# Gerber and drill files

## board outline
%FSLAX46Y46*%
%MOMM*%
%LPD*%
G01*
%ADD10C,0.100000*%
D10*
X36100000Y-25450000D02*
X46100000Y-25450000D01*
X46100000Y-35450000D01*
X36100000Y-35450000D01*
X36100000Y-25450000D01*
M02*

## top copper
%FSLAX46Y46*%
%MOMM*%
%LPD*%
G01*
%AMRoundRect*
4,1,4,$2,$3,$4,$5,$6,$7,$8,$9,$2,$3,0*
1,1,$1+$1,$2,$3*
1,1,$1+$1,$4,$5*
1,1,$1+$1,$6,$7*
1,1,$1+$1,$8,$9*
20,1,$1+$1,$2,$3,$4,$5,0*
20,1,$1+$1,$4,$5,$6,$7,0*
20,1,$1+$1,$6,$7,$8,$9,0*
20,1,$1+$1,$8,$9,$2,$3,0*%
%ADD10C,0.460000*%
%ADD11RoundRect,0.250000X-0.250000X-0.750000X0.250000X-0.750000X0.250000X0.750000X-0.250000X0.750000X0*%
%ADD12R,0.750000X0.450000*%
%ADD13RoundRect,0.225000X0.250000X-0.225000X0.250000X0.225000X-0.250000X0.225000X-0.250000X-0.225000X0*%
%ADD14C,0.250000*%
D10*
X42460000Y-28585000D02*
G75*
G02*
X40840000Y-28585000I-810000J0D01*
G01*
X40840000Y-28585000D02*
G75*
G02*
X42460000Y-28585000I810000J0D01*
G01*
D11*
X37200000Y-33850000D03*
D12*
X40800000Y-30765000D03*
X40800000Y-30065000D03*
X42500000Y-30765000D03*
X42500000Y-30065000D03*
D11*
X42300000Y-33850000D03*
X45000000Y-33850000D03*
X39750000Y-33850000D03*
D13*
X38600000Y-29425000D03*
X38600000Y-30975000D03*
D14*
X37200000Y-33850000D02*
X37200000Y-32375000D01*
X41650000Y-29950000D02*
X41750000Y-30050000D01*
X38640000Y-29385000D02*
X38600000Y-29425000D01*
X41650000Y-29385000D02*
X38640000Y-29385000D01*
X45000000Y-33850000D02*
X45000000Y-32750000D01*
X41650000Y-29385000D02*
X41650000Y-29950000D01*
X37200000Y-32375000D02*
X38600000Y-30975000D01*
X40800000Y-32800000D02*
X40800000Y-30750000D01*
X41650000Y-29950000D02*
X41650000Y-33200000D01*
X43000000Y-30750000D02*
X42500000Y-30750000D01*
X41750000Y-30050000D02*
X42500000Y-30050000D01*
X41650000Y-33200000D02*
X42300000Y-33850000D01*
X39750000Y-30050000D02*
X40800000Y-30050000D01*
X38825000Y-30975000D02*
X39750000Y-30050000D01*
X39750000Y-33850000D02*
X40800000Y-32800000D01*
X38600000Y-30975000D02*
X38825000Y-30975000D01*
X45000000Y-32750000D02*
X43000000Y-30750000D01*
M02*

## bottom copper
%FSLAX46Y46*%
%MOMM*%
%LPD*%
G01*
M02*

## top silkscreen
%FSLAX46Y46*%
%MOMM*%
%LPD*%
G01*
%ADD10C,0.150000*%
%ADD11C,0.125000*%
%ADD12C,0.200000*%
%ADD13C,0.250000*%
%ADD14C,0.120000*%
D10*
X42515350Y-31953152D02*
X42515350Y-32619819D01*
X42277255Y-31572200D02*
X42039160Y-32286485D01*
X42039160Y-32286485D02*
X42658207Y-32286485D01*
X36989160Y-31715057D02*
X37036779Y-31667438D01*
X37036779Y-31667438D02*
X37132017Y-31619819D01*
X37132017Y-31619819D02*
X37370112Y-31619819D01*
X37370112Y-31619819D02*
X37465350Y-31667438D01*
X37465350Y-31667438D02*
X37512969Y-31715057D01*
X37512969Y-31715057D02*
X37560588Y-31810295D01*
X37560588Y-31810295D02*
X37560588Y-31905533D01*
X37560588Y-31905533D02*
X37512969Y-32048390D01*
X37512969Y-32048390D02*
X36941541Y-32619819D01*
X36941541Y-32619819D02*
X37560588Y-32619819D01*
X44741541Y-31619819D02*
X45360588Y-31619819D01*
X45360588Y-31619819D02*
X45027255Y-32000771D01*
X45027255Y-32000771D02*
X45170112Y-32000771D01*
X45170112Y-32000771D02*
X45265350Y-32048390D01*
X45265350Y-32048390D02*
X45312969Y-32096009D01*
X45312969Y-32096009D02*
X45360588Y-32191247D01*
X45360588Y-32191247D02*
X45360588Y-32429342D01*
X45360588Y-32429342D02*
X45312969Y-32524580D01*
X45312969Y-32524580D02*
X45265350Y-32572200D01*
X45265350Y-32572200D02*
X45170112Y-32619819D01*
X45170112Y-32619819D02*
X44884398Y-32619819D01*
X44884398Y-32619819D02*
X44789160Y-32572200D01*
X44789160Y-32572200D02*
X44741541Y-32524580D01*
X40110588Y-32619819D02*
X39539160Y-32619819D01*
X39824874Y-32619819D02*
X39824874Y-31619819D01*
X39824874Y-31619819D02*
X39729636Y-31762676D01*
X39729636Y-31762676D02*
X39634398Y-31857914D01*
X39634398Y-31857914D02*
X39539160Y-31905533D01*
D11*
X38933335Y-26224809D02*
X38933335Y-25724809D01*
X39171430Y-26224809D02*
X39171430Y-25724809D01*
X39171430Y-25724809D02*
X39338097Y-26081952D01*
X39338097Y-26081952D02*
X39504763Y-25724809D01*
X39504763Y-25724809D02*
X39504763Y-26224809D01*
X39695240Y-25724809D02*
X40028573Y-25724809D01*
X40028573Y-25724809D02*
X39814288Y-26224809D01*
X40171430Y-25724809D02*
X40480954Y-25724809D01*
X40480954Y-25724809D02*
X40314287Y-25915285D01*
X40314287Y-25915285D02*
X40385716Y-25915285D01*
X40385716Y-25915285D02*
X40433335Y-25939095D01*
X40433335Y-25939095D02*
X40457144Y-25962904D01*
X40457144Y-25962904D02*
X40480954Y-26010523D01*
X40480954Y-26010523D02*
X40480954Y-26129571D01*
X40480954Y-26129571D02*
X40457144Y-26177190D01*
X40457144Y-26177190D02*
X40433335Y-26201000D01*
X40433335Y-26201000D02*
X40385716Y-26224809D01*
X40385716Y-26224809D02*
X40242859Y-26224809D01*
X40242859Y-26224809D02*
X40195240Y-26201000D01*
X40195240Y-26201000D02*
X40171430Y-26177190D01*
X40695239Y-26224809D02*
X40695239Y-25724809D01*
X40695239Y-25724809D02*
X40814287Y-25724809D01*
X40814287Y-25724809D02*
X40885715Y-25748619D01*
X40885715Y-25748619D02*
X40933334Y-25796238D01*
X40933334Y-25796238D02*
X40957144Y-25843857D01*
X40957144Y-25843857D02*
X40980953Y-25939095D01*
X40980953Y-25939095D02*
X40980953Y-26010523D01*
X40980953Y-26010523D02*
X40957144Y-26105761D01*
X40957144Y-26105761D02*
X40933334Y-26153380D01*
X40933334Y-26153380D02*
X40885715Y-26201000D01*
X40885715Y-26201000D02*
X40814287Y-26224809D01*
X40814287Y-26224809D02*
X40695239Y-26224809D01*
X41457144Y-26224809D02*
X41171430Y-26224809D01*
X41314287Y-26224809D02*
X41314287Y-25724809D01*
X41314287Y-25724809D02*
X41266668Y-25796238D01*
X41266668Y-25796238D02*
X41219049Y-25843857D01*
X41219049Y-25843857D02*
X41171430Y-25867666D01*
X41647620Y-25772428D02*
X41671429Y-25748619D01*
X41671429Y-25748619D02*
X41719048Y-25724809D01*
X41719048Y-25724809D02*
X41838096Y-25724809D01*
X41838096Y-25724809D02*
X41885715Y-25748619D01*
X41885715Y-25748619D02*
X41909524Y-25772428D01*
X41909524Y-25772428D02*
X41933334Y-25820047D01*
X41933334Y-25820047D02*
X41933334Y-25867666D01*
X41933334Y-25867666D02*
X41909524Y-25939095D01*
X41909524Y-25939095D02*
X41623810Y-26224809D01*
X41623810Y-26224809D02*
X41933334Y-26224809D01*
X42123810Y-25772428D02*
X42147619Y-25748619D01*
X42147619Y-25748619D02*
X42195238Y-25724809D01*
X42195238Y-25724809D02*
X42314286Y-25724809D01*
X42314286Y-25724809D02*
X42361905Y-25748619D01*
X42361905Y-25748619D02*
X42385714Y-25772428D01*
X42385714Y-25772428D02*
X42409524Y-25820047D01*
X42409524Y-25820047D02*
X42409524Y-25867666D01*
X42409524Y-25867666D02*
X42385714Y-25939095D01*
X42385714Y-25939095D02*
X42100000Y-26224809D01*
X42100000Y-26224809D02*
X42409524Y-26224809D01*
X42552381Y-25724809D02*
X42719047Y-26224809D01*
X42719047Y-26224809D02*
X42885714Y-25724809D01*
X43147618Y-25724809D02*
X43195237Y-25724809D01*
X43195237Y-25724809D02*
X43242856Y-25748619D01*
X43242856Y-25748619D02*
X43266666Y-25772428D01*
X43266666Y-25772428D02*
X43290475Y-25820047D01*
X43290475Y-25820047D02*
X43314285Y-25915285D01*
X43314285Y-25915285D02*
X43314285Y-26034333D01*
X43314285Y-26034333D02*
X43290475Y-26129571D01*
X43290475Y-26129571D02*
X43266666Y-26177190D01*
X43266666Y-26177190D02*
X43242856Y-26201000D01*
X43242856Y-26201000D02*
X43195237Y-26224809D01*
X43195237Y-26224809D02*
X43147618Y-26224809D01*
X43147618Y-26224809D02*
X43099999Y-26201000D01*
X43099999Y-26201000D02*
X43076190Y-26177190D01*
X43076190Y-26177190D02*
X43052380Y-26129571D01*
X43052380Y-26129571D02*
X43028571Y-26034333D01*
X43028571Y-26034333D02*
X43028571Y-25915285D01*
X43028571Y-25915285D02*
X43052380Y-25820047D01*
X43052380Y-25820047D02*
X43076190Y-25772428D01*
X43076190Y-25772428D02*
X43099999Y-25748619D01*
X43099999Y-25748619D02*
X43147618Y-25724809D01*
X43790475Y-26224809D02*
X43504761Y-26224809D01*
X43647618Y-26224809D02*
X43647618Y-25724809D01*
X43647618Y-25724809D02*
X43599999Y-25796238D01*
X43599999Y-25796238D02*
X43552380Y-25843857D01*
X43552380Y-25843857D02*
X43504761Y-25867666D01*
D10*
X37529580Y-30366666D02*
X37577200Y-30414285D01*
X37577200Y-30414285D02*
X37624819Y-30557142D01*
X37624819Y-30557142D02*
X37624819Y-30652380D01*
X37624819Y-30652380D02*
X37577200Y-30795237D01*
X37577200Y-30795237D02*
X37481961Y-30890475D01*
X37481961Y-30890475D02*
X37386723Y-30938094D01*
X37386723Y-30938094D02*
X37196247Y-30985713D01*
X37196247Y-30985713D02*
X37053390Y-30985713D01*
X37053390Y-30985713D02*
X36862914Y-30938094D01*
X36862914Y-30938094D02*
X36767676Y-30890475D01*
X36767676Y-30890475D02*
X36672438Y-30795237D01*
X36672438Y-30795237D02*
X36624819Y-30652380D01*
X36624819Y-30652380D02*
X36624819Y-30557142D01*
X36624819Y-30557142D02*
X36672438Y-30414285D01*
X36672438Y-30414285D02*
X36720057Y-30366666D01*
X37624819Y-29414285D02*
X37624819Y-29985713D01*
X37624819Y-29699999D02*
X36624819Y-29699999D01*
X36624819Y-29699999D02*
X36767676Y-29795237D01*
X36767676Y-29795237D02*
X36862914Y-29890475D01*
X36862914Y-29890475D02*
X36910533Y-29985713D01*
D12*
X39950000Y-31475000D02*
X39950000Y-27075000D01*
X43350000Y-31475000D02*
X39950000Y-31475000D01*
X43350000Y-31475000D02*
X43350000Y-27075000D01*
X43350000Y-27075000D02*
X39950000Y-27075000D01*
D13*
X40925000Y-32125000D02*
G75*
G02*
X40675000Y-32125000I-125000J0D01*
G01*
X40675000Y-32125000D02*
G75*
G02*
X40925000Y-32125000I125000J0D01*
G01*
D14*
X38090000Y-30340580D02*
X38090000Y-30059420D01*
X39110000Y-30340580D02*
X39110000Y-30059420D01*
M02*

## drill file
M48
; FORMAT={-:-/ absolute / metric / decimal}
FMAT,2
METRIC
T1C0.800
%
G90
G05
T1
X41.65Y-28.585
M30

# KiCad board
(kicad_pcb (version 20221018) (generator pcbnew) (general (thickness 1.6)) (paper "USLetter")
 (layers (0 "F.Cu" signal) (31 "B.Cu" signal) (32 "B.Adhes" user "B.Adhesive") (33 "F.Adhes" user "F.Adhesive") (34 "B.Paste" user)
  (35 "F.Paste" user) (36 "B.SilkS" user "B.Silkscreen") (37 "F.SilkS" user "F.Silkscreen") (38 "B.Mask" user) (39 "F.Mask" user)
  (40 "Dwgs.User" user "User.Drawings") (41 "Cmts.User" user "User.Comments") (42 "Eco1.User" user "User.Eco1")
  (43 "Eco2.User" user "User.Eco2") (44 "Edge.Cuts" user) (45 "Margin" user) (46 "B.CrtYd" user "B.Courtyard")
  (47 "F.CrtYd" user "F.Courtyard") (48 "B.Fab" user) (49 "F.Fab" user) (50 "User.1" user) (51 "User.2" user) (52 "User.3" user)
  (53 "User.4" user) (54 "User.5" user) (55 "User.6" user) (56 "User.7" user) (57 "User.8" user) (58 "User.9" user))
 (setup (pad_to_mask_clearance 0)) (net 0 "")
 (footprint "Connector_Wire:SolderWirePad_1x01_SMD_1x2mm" (layer "F.Cu") (at 37.2 33.85)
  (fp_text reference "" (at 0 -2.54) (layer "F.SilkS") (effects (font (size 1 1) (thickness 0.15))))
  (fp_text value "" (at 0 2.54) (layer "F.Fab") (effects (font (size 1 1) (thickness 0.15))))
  (pad "2" smd roundrect (at 0 0) (size 1 2) (layers "F.Cu" "F.Paste" "F.Mask") (roundrect_rratio 0.25)))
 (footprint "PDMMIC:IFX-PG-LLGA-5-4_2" (layer "F.Cu") (at 41.65 29.675 90)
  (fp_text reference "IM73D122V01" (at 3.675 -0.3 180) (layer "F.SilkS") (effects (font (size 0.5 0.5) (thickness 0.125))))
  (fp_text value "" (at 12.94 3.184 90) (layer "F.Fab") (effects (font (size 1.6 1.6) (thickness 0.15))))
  (fp_circle (center 1.09 0) (end 1.9 0) (stroke (width 0.46) (type solid)) (fill none) (layer "F.Cu"))
  (fp_line (start -1.8 -1.7) (end 2.6 -1.7) (stroke (width 0.2) (type solid)) (layer "F.SilkS"))
  (fp_line (start -1.8 1.7) (end -1.8 -1.7) (stroke (width 0.2) (type solid)) (layer "F.SilkS"))
  (fp_line (start -1.8 1.7) (end 2.6 1.7) (stroke (width 0.2) (type solid)) (layer "F.SilkS"))
  (fp_line (start 2.6 1.7) (end 2.6 -1.7) (stroke (width 0.2) (type solid)) (layer "F.SilkS"))
  (fp_circle (center -2.45 -0.85) (end -2.325 -0.85) (stroke (width 0.25) (type solid)) (fill none) (layer "F.SilkS"))
  (pad "" np_thru_hole circle (at 1.09 0 90) (size 0.8 0.8) (drill 0.8) (layers "F&B.Cu" "*.Mask"))
  (pad "1" smd rect (at -1.09 -0.85 90) (size 0.45 0.75) (layers "F.Cu" "F.Mask") (solder_mask_margin 0.102))
  (pad "2" smd rect (at -0.39 -0.85 90) (size 0.45 0.75) (layers "F.Cu" "F.Mask") (solder_mask_margin 0.102))
  (pad "3" smd rect (at -1.09 0.85 90) (size 0.45 0.75) (layers "F.Cu" "F.Mask") (solder_mask_margin 0.102))
  (pad "4" smd rect (at -0.39 0.85 90) (size 0.45 0.75) (layers "F.Cu" "F.Mask") (solder_mask_margin 0.102)))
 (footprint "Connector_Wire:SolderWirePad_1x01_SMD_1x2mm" (layer "F.Cu") (at 42.3 33.85)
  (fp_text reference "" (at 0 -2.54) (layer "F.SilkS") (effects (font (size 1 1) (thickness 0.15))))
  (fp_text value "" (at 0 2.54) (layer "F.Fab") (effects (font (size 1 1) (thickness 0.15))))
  (pad "4" smd roundrect (at 0 0) (size 1 2) (layers "F.Cu" "F.Paste" "F.Mask") (roundrect_rratio 0.25)))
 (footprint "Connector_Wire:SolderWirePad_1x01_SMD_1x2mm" (layer "F.Cu") (at 45 33.85)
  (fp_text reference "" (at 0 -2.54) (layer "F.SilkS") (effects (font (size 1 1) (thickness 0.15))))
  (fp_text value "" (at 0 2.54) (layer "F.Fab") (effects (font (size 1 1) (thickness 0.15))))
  (pad "3" smd roundrect (at 0 0) (size 1 2) (layers "F.Cu" "F.Paste" "F.Mask") (roundrect_rratio 0.25)))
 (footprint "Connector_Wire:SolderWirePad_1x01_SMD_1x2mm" (layer "F.Cu") (at 39.75 33.85)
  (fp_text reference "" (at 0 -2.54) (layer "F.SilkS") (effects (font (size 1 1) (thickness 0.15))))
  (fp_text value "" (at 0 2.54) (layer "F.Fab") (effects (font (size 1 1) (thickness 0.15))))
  (pad "1" smd roundrect (at 0 0) (size 1 2) (layers "F.Cu" "F.Paste" "F.Mask") (roundrect_rratio 0.25)))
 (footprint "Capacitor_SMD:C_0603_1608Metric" (layer "F.Cu") (at 38.6 30.2 90)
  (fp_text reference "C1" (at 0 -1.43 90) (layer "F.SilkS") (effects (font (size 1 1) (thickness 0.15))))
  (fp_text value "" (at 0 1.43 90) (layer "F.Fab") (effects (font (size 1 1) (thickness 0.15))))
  (fp_line (start -0.14058 -0.51) (end 0.14058 -0.51) (stroke (width 0.12) (type solid)) (layer "F.SilkS"))
  (fp_line (start -0.14058 0.51) (end 0.14058 0.51) (stroke (width 0.12) (type solid)) (layer "F.SilkS"))
  (pad "1" smd roundrect (at 0.775 0 90) (size 0.9 0.95) (layers "F.Cu" "F.Paste" "F.Mask") (roundrect_rratio 0.25))
  (pad "2" smd roundrect (at -0.775 0 90) (size 0.9 0.95) (layers "F.Cu" "F.Paste" "F.Mask") (roundrect_rratio 0.25)))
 (gr_rect (start 36.1 25.45) (end 46.1 35.45) (stroke (width 0.1) (type default)) (fill none) (layer "Edge.Cuts"))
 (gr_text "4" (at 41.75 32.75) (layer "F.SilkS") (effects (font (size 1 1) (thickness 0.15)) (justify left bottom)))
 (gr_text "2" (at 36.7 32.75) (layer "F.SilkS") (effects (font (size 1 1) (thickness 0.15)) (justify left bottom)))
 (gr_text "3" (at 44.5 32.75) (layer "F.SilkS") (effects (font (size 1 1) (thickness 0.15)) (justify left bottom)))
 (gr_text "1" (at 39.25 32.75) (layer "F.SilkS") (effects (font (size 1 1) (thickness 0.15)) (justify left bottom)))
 (segment (start 37.2 33.85) (end 37.2 32.375) (width 0.25) (layer "F.Cu") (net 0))
 (segment (start 41.65 29.95) (end 41.75 30.05) (width 0.25) (layer "F.Cu") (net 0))
 (segment (start 38.64 29.385) (end 38.6 29.425) (width 0.25) (layer "F.Cu") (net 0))
 (segment (start 41.65 29.385) (end 38.64 29.385) (width 0.25) (layer "F.Cu") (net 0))
 (segment (start 45 33.85) (end 45 32.75) (width 0.25) (layer "F.Cu") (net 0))
 (segment (start 41.65 29.385) (end 41.65 29.95) (width 0.25) (layer "F.Cu") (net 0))
 (segment (start 37.2 32.375) (end 38.6 30.975) (width 0.25) (layer "F.Cu") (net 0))
 (segment (start 40.8 32.8) (end 40.8 30.75) (width 0.25) (layer "F.Cu") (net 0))
 (segment (start 41.65 29.95) (end 41.65 33.2) (width 0.25) (layer "F.Cu") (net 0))
 (segment (start 43 30.75) (end 42.5 30.75) (width 0.25) (layer "F.Cu") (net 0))
 (segment (start 41.75 30.05) (end 42.5 30.05) (width 0.25) (layer "F.Cu") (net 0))
 (segment (start 41.65 33.2) (end 42.3 33.85) (width 0.25) (layer "F.Cu") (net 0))
 (segment (start 39.75 30.05) (end 40.8 30.05) (width 0.25) (layer "F.Cu") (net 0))
 (segment (start 38.825 30.975) (end 39.75 30.05) (width 0.25) (layer "F.Cu") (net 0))
 (segment (start 39.75 33.85) (end 40.8 32.8) (width 0.25) (layer "F.Cu") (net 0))
 (segment (start 38.6 30.975) (end 38.825 30.975) (width 0.25) (layer "F.Cu") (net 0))
 (segment (start 45 32.75) (end 43 30.75) (width 0.25) (layer "F.Cu") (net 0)))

